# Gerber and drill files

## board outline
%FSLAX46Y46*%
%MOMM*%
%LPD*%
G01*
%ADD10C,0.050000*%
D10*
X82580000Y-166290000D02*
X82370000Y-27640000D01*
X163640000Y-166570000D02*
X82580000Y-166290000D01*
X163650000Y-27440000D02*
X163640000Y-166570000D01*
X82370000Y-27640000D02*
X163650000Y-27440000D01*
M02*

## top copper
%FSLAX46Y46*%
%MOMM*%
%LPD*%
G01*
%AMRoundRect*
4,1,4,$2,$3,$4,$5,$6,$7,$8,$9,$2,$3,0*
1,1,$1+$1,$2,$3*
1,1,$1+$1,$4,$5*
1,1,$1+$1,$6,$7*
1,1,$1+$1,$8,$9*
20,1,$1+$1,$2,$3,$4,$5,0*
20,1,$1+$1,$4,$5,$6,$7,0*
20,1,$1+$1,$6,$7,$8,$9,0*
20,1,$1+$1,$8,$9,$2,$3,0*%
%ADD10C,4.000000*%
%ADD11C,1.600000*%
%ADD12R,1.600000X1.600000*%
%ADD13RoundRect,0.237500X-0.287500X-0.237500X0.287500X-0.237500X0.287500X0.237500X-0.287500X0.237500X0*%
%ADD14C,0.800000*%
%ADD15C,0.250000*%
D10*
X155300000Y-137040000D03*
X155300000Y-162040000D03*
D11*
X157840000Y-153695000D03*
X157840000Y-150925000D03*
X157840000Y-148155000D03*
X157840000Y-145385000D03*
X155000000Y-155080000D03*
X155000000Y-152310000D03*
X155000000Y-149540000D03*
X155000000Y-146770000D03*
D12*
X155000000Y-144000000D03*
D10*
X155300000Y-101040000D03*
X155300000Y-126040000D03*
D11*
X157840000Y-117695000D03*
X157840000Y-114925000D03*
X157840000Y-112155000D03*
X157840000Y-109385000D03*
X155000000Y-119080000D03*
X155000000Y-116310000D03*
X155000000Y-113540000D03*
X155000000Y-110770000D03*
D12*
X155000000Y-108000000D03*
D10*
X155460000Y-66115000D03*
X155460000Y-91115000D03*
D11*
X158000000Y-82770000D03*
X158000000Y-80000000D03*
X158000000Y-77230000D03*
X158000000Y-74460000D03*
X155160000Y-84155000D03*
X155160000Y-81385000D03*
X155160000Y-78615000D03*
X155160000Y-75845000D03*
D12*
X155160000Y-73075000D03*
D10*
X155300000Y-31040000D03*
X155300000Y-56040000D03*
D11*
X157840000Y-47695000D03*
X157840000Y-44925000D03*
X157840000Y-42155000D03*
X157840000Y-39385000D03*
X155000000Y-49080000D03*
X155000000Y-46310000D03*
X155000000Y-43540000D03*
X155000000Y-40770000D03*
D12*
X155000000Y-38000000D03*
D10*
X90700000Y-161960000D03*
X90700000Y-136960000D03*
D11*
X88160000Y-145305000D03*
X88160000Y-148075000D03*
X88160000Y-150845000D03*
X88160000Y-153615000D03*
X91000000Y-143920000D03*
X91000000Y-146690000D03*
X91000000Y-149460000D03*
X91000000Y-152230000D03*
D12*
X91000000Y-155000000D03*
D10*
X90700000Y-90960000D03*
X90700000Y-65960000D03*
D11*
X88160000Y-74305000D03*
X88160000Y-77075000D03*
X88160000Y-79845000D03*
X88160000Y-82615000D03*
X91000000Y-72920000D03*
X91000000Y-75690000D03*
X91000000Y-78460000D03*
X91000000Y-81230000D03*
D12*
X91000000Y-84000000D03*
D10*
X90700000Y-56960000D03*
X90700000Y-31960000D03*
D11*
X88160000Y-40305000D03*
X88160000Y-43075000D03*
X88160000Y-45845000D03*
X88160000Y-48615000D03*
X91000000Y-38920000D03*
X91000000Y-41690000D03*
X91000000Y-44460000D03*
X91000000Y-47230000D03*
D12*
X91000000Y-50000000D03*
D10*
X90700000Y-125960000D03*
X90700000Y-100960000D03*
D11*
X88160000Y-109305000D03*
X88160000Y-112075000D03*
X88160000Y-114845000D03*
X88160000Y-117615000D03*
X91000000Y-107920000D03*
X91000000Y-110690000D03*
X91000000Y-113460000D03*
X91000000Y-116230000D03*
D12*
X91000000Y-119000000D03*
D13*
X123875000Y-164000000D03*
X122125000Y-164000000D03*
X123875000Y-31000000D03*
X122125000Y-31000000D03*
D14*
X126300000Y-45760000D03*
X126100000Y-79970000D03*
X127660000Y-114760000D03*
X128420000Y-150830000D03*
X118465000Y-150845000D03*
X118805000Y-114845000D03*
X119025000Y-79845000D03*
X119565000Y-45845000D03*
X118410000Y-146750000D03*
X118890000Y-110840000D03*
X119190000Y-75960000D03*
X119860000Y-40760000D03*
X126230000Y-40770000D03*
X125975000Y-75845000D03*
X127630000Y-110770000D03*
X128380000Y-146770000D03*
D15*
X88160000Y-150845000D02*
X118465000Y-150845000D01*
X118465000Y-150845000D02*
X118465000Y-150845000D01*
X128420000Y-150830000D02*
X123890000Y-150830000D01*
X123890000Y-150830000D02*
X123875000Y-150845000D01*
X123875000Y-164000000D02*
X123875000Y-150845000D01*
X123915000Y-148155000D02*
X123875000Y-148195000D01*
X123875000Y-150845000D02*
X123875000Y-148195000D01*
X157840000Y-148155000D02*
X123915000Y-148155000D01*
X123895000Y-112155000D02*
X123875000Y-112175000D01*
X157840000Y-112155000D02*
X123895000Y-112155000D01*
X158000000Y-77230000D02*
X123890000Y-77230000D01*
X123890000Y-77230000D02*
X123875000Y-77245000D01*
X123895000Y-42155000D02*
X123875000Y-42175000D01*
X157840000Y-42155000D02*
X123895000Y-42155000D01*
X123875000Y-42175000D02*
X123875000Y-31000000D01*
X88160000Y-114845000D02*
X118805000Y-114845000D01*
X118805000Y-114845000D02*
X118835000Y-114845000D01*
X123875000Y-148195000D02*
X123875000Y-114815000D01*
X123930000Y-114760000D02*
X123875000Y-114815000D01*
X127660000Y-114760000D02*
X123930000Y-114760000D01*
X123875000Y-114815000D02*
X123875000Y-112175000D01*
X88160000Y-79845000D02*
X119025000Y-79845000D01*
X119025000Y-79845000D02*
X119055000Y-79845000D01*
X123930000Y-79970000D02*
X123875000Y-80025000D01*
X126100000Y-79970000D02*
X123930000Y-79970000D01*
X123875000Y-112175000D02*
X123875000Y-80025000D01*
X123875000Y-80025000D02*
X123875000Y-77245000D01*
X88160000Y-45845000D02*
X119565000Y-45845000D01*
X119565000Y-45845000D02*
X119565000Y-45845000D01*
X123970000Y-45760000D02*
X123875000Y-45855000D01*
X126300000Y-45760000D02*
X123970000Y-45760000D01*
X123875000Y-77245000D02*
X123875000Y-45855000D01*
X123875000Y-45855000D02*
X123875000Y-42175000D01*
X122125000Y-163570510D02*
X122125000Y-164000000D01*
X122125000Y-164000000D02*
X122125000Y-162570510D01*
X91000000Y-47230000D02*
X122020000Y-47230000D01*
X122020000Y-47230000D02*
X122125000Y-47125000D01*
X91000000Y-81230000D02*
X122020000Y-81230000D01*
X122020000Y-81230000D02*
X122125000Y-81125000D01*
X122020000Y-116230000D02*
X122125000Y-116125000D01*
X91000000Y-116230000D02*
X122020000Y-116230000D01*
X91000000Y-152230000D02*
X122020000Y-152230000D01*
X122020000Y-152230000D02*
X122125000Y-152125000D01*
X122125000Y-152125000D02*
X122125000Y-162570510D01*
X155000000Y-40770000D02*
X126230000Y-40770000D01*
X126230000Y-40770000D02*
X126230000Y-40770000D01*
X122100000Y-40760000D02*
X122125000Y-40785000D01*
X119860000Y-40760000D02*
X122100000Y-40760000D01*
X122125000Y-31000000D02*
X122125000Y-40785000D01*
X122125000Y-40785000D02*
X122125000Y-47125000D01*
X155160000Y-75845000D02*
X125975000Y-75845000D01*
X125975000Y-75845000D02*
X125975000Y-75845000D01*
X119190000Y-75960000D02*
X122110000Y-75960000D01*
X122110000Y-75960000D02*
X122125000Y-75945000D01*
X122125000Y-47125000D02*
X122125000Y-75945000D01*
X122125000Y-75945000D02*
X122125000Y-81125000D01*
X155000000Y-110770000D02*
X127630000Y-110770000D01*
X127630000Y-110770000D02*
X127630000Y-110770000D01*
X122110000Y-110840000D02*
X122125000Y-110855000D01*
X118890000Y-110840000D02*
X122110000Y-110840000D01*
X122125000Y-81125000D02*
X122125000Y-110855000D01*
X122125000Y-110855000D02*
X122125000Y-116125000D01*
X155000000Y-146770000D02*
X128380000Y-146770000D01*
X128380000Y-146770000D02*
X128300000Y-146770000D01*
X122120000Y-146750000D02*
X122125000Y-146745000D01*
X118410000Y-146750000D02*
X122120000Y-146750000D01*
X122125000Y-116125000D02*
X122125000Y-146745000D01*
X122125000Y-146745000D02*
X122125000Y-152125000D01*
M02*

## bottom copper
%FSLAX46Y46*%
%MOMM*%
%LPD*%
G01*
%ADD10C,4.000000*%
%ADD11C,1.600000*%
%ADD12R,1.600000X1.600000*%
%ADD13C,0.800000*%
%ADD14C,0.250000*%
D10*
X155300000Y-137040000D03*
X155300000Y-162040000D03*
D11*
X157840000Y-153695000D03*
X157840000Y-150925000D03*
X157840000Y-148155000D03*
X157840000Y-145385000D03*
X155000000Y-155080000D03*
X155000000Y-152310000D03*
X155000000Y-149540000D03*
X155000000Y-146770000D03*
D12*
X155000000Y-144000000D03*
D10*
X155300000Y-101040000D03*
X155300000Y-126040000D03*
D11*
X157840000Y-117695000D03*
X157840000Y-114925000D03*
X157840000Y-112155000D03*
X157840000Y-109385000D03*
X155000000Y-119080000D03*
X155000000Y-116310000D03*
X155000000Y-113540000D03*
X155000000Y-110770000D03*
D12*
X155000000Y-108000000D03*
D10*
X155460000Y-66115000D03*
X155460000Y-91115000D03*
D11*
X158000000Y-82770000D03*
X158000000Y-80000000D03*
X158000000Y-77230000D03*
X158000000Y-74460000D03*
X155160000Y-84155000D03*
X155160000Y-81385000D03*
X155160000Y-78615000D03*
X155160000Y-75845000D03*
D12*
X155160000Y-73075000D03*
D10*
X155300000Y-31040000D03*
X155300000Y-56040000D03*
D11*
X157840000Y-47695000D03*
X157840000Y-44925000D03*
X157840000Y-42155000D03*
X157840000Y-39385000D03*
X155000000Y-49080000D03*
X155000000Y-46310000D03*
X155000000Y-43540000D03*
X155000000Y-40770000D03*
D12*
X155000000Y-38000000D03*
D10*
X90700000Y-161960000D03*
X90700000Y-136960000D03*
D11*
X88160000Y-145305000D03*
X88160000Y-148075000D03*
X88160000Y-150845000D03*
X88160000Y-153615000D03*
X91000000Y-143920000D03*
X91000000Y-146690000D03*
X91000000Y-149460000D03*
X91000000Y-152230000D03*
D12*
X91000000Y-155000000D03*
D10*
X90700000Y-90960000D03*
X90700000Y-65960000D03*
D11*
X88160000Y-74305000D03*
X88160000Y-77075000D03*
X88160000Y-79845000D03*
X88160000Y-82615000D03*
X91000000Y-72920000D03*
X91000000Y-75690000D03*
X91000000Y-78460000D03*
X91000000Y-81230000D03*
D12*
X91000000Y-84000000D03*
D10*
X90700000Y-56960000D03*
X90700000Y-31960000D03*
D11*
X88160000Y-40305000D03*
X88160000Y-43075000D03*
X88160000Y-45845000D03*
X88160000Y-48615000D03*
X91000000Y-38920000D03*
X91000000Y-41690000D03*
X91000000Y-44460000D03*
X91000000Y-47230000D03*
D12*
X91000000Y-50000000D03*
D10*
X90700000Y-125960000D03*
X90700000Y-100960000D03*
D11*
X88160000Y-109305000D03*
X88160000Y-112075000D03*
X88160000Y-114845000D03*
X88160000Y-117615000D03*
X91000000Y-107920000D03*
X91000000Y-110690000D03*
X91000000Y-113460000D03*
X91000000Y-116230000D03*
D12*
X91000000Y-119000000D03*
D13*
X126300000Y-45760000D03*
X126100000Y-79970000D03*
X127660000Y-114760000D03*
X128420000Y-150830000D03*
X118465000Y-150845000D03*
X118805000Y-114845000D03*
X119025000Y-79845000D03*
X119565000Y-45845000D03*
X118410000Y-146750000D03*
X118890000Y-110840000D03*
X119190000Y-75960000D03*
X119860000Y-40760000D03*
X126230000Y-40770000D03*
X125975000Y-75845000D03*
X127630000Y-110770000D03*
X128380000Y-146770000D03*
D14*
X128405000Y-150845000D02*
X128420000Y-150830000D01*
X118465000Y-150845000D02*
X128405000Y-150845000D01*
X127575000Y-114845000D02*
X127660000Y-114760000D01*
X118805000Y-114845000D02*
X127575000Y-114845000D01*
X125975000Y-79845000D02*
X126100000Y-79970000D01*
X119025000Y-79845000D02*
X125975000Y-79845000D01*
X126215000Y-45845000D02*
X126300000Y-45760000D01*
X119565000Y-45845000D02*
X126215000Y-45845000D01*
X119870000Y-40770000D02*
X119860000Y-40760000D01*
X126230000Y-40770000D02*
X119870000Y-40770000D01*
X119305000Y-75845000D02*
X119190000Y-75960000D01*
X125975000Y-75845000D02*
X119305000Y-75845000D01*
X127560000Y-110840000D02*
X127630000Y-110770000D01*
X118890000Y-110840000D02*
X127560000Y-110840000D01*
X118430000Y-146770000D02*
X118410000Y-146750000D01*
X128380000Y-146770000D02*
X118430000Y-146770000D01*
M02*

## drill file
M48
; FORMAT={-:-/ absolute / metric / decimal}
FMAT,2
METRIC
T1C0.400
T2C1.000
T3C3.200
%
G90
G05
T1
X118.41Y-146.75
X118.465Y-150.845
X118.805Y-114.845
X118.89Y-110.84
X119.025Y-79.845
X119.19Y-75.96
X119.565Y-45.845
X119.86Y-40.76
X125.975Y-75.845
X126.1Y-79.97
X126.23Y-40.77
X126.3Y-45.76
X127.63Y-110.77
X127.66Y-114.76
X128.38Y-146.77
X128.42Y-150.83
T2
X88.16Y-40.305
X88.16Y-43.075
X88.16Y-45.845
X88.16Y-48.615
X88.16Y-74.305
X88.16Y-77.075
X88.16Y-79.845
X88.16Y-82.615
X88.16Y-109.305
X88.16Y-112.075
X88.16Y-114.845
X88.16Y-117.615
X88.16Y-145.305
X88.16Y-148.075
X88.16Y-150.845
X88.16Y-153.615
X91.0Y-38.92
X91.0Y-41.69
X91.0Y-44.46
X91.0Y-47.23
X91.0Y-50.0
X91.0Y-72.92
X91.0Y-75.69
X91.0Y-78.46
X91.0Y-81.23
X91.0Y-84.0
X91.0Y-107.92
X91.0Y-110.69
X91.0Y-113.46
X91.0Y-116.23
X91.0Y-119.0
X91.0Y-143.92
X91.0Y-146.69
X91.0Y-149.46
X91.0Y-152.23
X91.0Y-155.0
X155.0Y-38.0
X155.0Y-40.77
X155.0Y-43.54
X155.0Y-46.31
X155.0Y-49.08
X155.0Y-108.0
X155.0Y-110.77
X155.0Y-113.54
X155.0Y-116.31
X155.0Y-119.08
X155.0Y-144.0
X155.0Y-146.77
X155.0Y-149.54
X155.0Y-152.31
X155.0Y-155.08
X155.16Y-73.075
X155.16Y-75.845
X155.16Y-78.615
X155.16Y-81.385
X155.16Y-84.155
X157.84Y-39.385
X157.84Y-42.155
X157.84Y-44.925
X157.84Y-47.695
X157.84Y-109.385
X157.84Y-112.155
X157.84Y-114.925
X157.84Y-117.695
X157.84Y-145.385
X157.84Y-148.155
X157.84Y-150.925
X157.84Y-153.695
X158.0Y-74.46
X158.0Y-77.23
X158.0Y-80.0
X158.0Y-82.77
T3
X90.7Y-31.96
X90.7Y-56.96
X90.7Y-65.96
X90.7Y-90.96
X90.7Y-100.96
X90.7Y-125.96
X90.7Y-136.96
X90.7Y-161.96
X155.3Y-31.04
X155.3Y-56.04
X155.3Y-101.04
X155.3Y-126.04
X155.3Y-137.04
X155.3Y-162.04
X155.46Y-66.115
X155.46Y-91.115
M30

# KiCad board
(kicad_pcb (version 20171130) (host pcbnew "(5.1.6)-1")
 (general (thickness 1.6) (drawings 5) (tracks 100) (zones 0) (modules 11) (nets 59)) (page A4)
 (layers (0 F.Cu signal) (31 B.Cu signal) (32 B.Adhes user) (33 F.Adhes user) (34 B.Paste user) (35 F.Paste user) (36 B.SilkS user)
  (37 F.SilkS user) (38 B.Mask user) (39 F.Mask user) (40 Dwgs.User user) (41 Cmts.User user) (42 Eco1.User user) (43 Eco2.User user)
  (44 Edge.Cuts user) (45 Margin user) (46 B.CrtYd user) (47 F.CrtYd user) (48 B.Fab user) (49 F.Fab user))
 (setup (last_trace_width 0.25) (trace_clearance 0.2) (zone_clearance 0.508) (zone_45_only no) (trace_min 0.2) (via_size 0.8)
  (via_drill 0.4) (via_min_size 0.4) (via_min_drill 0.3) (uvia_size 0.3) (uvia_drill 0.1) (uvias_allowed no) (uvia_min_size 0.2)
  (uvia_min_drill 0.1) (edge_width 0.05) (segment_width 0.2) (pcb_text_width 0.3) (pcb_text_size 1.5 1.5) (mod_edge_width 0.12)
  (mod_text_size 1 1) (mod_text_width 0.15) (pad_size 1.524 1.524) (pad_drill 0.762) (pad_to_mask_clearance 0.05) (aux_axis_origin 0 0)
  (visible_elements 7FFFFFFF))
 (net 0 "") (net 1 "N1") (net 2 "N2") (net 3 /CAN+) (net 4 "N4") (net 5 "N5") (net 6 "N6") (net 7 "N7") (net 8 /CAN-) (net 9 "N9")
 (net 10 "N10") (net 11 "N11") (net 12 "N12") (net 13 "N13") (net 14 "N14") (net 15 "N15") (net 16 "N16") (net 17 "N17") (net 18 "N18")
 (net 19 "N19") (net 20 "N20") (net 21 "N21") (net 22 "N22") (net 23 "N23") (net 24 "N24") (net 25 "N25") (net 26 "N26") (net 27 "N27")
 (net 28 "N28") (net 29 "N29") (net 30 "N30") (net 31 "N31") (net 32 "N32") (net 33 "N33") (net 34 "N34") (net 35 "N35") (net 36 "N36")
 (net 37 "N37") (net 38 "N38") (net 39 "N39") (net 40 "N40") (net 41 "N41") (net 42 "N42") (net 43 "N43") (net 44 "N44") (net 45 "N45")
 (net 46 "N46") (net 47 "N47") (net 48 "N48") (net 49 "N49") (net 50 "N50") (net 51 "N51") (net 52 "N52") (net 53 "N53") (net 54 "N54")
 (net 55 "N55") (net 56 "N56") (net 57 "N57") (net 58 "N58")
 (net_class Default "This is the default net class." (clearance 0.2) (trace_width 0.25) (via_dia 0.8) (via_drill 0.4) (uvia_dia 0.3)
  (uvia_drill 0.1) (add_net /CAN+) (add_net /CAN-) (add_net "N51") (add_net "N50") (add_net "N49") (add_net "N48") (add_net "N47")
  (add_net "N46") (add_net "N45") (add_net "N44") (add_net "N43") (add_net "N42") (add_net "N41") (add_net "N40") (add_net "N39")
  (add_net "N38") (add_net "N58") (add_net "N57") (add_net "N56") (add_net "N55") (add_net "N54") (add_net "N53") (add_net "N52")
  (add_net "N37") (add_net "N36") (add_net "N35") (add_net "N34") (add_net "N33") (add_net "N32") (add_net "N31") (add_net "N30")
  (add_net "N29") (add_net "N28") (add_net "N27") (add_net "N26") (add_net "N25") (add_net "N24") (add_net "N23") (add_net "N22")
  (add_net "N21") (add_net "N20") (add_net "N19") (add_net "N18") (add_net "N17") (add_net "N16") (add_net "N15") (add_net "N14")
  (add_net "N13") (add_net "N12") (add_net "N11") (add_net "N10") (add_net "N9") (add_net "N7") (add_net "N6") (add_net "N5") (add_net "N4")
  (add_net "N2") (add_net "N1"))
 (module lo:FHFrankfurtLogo (layer F.Cu) (at 122.29 88.09)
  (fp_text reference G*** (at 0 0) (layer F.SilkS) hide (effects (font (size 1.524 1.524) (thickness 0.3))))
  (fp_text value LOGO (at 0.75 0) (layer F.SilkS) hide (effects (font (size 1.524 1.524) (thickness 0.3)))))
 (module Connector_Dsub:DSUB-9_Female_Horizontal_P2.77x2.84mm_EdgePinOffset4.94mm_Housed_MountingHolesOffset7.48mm (layer F.Cu)
  (at 155 144 90)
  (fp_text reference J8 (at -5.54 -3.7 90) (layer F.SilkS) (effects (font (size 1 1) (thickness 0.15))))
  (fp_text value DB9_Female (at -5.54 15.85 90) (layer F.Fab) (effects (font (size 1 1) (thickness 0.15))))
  (pad 0 thru_hole circle (at 6.96 0.3 90) (size 4 4) (drill 3.2) (layers *.Cu *.Mask))
  (pad 0 thru_hole circle (at -18.04 0.3 90) (size 4 4) (drill 3.2) (layers *.Cu *.Mask))
  (pad 9 thru_hole circle (at -9.695 2.84 90) (size 1.6 1.6) (drill 1) (layers *.Cu *.Mask) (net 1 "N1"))
  (pad 8 thru_hole circle (at -6.925 2.84 90) (size 1.6 1.6) (drill 1) (layers *.Cu *.Mask) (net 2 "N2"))
  (pad 7 thru_hole circle (at -4.155 2.84 90) (size 1.6 1.6) (drill 1) (layers *.Cu *.Mask) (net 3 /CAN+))
  (pad 6 thru_hole circle (at -1.385 2.84 90) (size 1.6 1.6) (drill 1) (layers *.Cu *.Mask) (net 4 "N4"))
  (pad 5 thru_hole circle (at -11.08 0 90) (size 1.6 1.6) (drill 1) (layers *.Cu *.Mask) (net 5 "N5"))
  (pad 4 thru_hole circle (at -8.31 0 90) (size 1.6 1.6) (drill 1) (layers *.Cu *.Mask) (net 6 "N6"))
  (pad 3 thru_hole circle (at -5.54 0 90) (size 1.6 1.6) (drill 1) (layers *.Cu *.Mask) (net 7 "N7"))
  (pad 2 thru_hole circle (at -2.77 0 90) (size 1.6 1.6) (drill 1) (layers *.Cu *.Mask) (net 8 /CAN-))
  (pad 1 thru_hole rect (at 0 0 90) (size 1.6 1.6) (drill 1) (layers *.Cu *.Mask) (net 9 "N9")))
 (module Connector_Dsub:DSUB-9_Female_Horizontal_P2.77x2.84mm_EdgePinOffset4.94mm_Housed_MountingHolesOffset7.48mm (layer F.Cu)
  (at 155 108 90)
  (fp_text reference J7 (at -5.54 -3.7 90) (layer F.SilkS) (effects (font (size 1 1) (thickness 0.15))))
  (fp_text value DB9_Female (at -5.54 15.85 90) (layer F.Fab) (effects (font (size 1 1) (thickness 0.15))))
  (pad 0 thru_hole circle (at 6.96 0.3 90) (size 4 4) (drill 3.2) (layers *.Cu *.Mask))
  (pad 0 thru_hole circle (at -18.04 0.3 90) (size 4 4) (drill 3.2) (layers *.Cu *.Mask))
  (pad 9 thru_hole circle (at -9.695 2.84 90) (size 1.6 1.6) (drill 1) (layers *.Cu *.Mask) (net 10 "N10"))
  (pad 8 thru_hole circle (at -6.925 2.84 90) (size 1.6 1.6) (drill 1) (layers *.Cu *.Mask) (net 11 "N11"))
  (pad 7 thru_hole circle (at -4.155 2.84 90) (size 1.6 1.6) (drill 1) (layers *.Cu *.Mask) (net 3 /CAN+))
  (pad 6 thru_hole circle (at -1.385 2.84 90) (size 1.6 1.6) (drill 1) (layers *.Cu *.Mask) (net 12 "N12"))
  (pad 5 thru_hole circle (at -11.08 0 90) (size 1.6 1.6) (drill 1) (layers *.Cu *.Mask) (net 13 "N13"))
  (pad 4 thru_hole circle (at -8.31 0 90) (size 1.6 1.6) (drill 1) (layers *.Cu *.Mask) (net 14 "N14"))
  (pad 3 thru_hole circle (at -5.54 0 90) (size 1.6 1.6) (drill 1) (layers *.Cu *.Mask) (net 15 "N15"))
  (pad 2 thru_hole circle (at -2.77 0 90) (size 1.6 1.6) (drill 1) (layers *.Cu *.Mask) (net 8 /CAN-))
  (pad 1 thru_hole rect (at 0 0 90) (size 1.6 1.6) (drill 1) (layers *.Cu *.Mask) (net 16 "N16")))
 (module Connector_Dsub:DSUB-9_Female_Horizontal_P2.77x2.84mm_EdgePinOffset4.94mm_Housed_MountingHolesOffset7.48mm (layer F.Cu)
  (at 155.16 73.075 90)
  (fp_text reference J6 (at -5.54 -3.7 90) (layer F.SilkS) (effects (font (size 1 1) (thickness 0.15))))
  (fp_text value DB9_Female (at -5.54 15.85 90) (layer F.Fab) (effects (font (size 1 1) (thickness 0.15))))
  (pad 0 thru_hole circle (at 6.96 0.3 90) (size 4 4) (drill 3.2) (layers *.Cu *.Mask))
  (pad 0 thru_hole circle (at -18.04 0.3 90) (size 4 4) (drill 3.2) (layers *.Cu *.Mask))
  (pad 9 thru_hole circle (at -9.695 2.84 90) (size 1.6 1.6) (drill 1) (layers *.Cu *.Mask) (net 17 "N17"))
  (pad 8 thru_hole circle (at -6.925 2.84 90) (size 1.6 1.6) (drill 1) (layers *.Cu *.Mask) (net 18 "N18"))
  (pad 7 thru_hole circle (at -4.155 2.84 90) (size 1.6 1.6) (drill 1) (layers *.Cu *.Mask) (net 3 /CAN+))
  (pad 6 thru_hole circle (at -1.385 2.84 90) (size 1.6 1.6) (drill 1) (layers *.Cu *.Mask) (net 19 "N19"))
  (pad 5 thru_hole circle (at -11.08 0 90) (size 1.6 1.6) (drill 1) (layers *.Cu *.Mask) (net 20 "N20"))
  (pad 4 thru_hole circle (at -8.31 0 90) (size 1.6 1.6) (drill 1) (layers *.Cu *.Mask) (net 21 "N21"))
  (pad 3 thru_hole circle (at -5.54 0 90) (size 1.6 1.6) (drill 1) (layers *.Cu *.Mask) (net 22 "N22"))
  (pad 2 thru_hole circle (at -2.77 0 90) (size 1.6 1.6) (drill 1) (layers *.Cu *.Mask) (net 8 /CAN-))
  (pad 1 thru_hole rect (at 0 0 90) (size 1.6 1.6) (drill 1) (layers *.Cu *.Mask) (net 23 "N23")))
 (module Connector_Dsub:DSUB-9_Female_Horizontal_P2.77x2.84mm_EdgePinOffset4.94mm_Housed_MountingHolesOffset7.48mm (layer F.Cu)
  (at 155 38 90)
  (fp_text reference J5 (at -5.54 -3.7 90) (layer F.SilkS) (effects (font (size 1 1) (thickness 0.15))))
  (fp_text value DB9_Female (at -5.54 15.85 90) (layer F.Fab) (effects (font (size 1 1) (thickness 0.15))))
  (pad 0 thru_hole circle (at 6.96 0.3 90) (size 4 4) (drill 3.2) (layers *.Cu *.Mask))
  (pad 0 thru_hole circle (at -18.04 0.3 90) (size 4 4) (drill 3.2) (layers *.Cu *.Mask))
  (pad 9 thru_hole circle (at -9.695 2.84 90) (size 1.6 1.6) (drill 1) (layers *.Cu *.Mask) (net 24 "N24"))
  (pad 8 thru_hole circle (at -6.925 2.84 90) (size 1.6 1.6) (drill 1) (layers *.Cu *.Mask) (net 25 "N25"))
  (pad 7 thru_hole circle (at -4.155 2.84 90) (size 1.6 1.6) (drill 1) (layers *.Cu *.Mask) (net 3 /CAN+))
  (pad 6 thru_hole circle (at -1.385 2.84 90) (size 1.6 1.6) (drill 1) (layers *.Cu *.Mask) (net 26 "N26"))
  (pad 5 thru_hole circle (at -11.08 0 90) (size 1.6 1.6) (drill 1) (layers *.Cu *.Mask) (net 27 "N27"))
  (pad 4 thru_hole circle (at -8.31 0 90) (size 1.6 1.6) (drill 1) (layers *.Cu *.Mask) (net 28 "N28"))
  (pad 3 thru_hole circle (at -5.54 0 90) (size 1.6 1.6) (drill 1) (layers *.Cu *.Mask) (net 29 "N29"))
  (pad 2 thru_hole circle (at -2.77 0 90) (size 1.6 1.6) (drill 1) (layers *.Cu *.Mask) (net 8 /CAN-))
  (pad 1 thru_hole rect (at 0 0 90) (size 1.6 1.6) (drill 1) (layers *.Cu *.Mask) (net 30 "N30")))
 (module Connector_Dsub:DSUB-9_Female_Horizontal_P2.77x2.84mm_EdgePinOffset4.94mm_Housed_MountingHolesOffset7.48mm (layer F.Cu)
  (at 91 155 270)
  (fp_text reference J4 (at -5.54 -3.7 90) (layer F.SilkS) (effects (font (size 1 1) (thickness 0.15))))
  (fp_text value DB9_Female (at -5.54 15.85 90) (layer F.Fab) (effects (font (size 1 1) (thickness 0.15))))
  (pad 0 thru_hole circle (at 6.96 0.3 270) (size 4 4) (drill 3.2) (layers *.Cu *.Mask))
  (pad 0 thru_hole circle (at -18.04 0.3 270) (size 4 4) (drill 3.2) (layers *.Cu *.Mask))
  (pad 9 thru_hole circle (at -9.695 2.84 270) (size 1.6 1.6) (drill 1) (layers *.Cu *.Mask) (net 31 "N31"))
  (pad 8 thru_hole circle (at -6.925 2.84 270) (size 1.6 1.6) (drill 1) (layers *.Cu *.Mask) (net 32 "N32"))
  (pad 7 thru_hole circle (at -4.155 2.84 270) (size 1.6 1.6) (drill 1) (layers *.Cu *.Mask) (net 3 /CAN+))
  (pad 6 thru_hole circle (at -1.385 2.84 270) (size 1.6 1.6) (drill 1) (layers *.Cu *.Mask) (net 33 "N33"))
  (pad 5 thru_hole circle (at -11.08 0 270) (size 1.6 1.6) (drill 1) (layers *.Cu *.Mask) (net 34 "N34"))
  (pad 4 thru_hole circle (at -8.31 0 270) (size 1.6 1.6) (drill 1) (layers *.Cu *.Mask) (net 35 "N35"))
  (pad 3 thru_hole circle (at -5.54 0 270) (size 1.6 1.6) (drill 1) (layers *.Cu *.Mask) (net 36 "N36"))
  (pad 2 thru_hole circle (at -2.77 0 270) (size 1.6 1.6) (drill 1) (layers *.Cu *.Mask) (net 8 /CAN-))
  (pad 1 thru_hole rect (at 0 0 270) (size 1.6 1.6) (drill 1) (layers *.Cu *.Mask) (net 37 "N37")))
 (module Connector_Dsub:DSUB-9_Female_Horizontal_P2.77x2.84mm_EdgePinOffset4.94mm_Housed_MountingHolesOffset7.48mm (layer F.Cu)
  (at 91 84 270)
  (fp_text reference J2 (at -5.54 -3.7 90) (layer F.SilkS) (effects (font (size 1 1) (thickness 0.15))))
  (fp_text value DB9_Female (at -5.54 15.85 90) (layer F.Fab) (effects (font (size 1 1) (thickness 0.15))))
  (pad 0 thru_hole circle (at 6.96 0.3 270) (size 4 4) (drill 3.2) (layers *.Cu *.Mask))
  (pad 0 thru_hole circle (at -18.04 0.3 270) (size 4 4) (drill 3.2) (layers *.Cu *.Mask))
  (pad 9 thru_hole circle (at -9.695 2.84 270) (size 1.6 1.6) (drill 1) (layers *.Cu *.Mask) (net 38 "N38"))
  (pad 8 thru_hole circle (at -6.925 2.84 270) (size 1.6 1.6) (drill 1) (layers *.Cu *.Mask) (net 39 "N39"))
  (pad 7 thru_hole circle (at -4.155 2.84 270) (size 1.6 1.6) (drill 1) (layers *.Cu *.Mask) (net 3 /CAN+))
  (pad 6 thru_hole circle (at -1.385 2.84 270) (size 1.6 1.6) (drill 1) (layers *.Cu *.Mask) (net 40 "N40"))
  (pad 5 thru_hole circle (at -11.08 0 270) (size 1.6 1.6) (drill 1) (layers *.Cu *.Mask) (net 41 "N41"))
  (pad 4 thru_hole circle (at -8.31 0 270) (size 1.6 1.6) (drill 1) (layers *.Cu *.Mask) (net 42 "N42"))
  (pad 3 thru_hole circle (at -5.54 0 270) (size 1.6 1.6) (drill 1) (layers *.Cu *.Mask) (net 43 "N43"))
  (pad 2 thru_hole circle (at -2.77 0 270) (size 1.6 1.6) (drill 1) (layers *.Cu *.Mask) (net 8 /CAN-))
  (pad 1 thru_hole rect (at 0 0 270) (size 1.6 1.6) (drill 1) (layers *.Cu *.Mask) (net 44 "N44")))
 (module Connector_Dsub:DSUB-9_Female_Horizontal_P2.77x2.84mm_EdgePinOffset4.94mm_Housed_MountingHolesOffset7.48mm (layer F.Cu)
  (at 91 50 270)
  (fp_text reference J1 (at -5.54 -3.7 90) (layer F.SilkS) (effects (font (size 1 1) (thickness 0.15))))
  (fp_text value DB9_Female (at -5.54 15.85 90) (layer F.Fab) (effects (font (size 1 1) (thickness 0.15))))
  (pad 0 thru_hole circle (at 6.96 0.3 270) (size 4 4) (drill 3.2) (layers *.Cu *.Mask))
  (pad 0 thru_hole circle (at -18.04 0.3 270) (size 4 4) (drill 3.2) (layers *.Cu *.Mask))
  (pad 9 thru_hole circle (at -9.695 2.84 270) (size 1.6 1.6) (drill 1) (layers *.Cu *.Mask) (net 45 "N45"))
  (pad 8 thru_hole circle (at -6.925 2.84 270) (size 1.6 1.6) (drill 1) (layers *.Cu *.Mask) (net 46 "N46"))
  (pad 7 thru_hole circle (at -4.155 2.84 270) (size 1.6 1.6) (drill 1) (layers *.Cu *.Mask) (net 3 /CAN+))
  (pad 6 thru_hole circle (at -1.385 2.84 270) (size 1.6 1.6) (drill 1) (layers *.Cu *.Mask) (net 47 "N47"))
  (pad 5 thru_hole circle (at -11.08 0 270) (size 1.6 1.6) (drill 1) (layers *.Cu *.Mask) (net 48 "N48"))
  (pad 4 thru_hole circle (at -8.31 0 270) (size 1.6 1.6) (drill 1) (layers *.Cu *.Mask) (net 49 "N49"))
  (pad 3 thru_hole circle (at -5.54 0 270) (size 1.6 1.6) (drill 1) (layers *.Cu *.Mask) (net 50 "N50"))
  (pad 2 thru_hole circle (at -2.77 0 270) (size 1.6 1.6) (drill 1) (layers *.Cu *.Mask) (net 8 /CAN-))
  (pad 1 thru_hole rect (at 0 0 270) (size 1.6 1.6) (drill 1) (layers *.Cu *.Mask) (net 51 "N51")))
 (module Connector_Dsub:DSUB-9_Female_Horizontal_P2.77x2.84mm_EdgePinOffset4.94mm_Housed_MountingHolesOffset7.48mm (layer F.Cu)
  (at 91 119 270)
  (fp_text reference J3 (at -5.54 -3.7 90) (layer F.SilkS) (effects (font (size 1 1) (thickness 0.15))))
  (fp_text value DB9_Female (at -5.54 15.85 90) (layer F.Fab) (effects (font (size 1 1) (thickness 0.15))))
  (pad 0 thru_hole circle (at 6.96 0.3 270) (size 4 4) (drill 3.2) (layers *.Cu *.Mask))
  (pad 0 thru_hole circle (at -18.04 0.3 270) (size 4 4) (drill 3.2) (layers *.Cu *.Mask))
  (pad 9 thru_hole circle (at -9.695 2.84 270) (size 1.6 1.6) (drill 1) (layers *.Cu *.Mask) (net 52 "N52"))
  (pad 8 thru_hole circle (at -6.925 2.84 270) (size 1.6 1.6) (drill 1) (layers *.Cu *.Mask) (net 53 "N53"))
  (pad 7 thru_hole circle (at -4.155 2.84 270) (size 1.6 1.6) (drill 1) (layers *.Cu *.Mask) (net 3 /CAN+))
  (pad 6 thru_hole circle (at -1.385 2.84 270) (size 1.6 1.6) (drill 1) (layers *.Cu *.Mask) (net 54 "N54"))
  (pad 5 thru_hole circle (at -11.08 0 270) (size 1.6 1.6) (drill 1) (layers *.Cu *.Mask) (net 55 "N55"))
  (pad 4 thru_hole circle (at -8.31 0 270) (size 1.6 1.6) (drill 1) (layers *.Cu *.Mask) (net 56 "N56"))
  (pad 3 thru_hole circle (at -5.54 0 270) (size 1.6 1.6) (drill 1) (layers *.Cu *.Mask) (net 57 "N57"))
  (pad 2 thru_hole circle (at -2.77 0 270) (size 1.6 1.6) (drill 1) (layers *.Cu *.Mask) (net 8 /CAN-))
  (pad 1 thru_hole rect (at 0 0 270) (size 1.6 1.6) (drill 1) (layers *.Cu *.Mask) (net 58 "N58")))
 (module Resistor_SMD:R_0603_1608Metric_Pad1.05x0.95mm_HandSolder (layer F.Cu) (at 123 164)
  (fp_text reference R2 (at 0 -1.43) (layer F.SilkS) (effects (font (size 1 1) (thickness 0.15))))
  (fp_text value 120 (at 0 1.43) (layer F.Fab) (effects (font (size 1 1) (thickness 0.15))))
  (pad 2 smd roundrect (at 0.875 0) (size 1.05 0.95) (layers F.Cu F.Paste F.Mask) (roundrect_rratio 0.25) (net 3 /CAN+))
  (pad 1 smd roundrect (at -0.875 0) (size 1.05 0.95) (layers F.Cu F.Paste F.Mask) (roundrect_rratio 0.25) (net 8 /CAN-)))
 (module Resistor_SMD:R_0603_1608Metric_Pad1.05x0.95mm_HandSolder (layer F.Cu) (at 123 31)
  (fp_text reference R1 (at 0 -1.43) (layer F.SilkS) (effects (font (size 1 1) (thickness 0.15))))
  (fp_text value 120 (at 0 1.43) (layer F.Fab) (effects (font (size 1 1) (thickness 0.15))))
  (pad 2 smd roundrect (at 0.875 0) (size 1.05 0.95) (layers F.Cu F.Paste F.Mask) (roundrect_rratio 0.25) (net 3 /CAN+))
  (pad 1 smd roundrect (at -0.875 0) (size 1.05 0.95) (layers F.Cu F.Paste F.Mask) (roundrect_rratio 0.25) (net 8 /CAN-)))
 (gr_line (start 82.58 166.29) (end 82.37 27.64) (layer Edge.Cuts) (width 0.05))
 (gr_line (start 163.64 166.57) (end 82.58 166.29) (layer Edge.Cuts) (width 0.05))
 (gr_line (start 163.65 27.44) (end 163.64 166.57) (layer Edge.Cuts) (width 0.05))
 (gr_line (start 82.37 27.64) (end 163.65 27.44) (layer Edge.Cuts) (width 0.05))
 (via (at 126.3 45.76) (size 0.8) (drill 0.4) (layers F.Cu B.Cu) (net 3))
 (via (at 126.1 79.97) (size 0.8) (drill 0.4) (layers F.Cu B.Cu) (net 3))
 (via (at 127.66 114.76) (size 0.8) (drill 0.4) (layers F.Cu B.Cu) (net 3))
 (via (at 128.42 150.83) (size 0.8) (drill 0.4) (layers F.Cu B.Cu) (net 3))
 (segment (start 88.16 150.845) (end 118.465 150.845) (width 0.25) (layer F.Cu) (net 3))
 (segment (start 118.465 150.845) (end 118.465 150.845) (width 0.25) (layer F.Cu) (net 3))
 (via (at 118.465 150.845) (size 0.8) (drill 0.4) (layers F.Cu B.Cu) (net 3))
 (segment (start 128.405 150.845) (end 128.42 150.83) (width 0.25) (layer B.Cu) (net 3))
 (segment (start 118.465 150.845) (end 128.405 150.845) (width 0.25) (layer B.Cu) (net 3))
 (segment (start 128.42 150.83) (end 123.89 150.83) (width 0.25) (layer F.Cu) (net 3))
 (segment (start 123.89 150.83) (end 123.875 150.845) (width 0.25) (layer F.Cu) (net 3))
 (segment (start 123.875 164) (end 123.875 150.845) (width 0.25) (layer F.Cu) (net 3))
 (segment (start 123.915 148.155) (end 123.875 148.195) (width 0.25) (layer F.Cu) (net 3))
 (segment (start 123.875 150.845) (end 123.875 148.195) (width 0.25) (layer F.Cu) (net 3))
 (segment (start 157.84 148.155) (end 123.915 148.155) (width 0.25) (layer F.Cu) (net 3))
 (segment (start 123.895 112.155) (end 123.875 112.175) (width 0.25) (layer F.Cu) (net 3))
 (segment (start 157.84 112.155) (end 123.895 112.155) (width 0.25) (layer F.Cu) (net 3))
 (segment (start 158 77.23) (end 123.89 77.23) (width 0.25) (layer F.Cu) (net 3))
 (segment (start 123.89 77.23) (end 123.875 77.245) (width 0.25) (layer F.Cu) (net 3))
 (segment (start 123.895 42.155) (end 123.875 42.175) (width 0.25) (layer F.Cu) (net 3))
 (segment (start 157.84 42.155) (end 123.895 42.155) (width 0.25) (layer F.Cu) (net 3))
 (segment (start 123.875 42.175) (end 123.875 31) (width 0.25) (layer F.Cu) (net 3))
 (segment (start 88.16 114.845) (end 118.805 114.845) (width 0.25) (layer F.Cu) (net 3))
 (segment (start 118.805 114.845) (end 118.835 114.845) (width 0.25) (layer F.Cu) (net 3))
 (via (at 118.805 114.845) (size 0.8) (drill 0.4) (layers F.Cu B.Cu) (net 3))
 (segment (start 127.575 114.845) (end 127.66 114.76) (width 0.25) (layer B.Cu) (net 3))
 (segment (start 118.805 114.845) (end 127.575 114.845) (width 0.25) (layer B.Cu) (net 3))
 (segment (start 123.875 148.195) (end 123.875 114.815) (width 0.25) (layer F.Cu) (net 3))
 (segment (start 123.93 114.76) (end 123.875 114.815) (width 0.25) (layer F.Cu) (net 3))
 (segment (start 127.66 114.76) (end 123.93 114.76) (width 0.25) (layer F.Cu) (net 3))
 (segment (start 123.875 114.815) (end 123.875 112.175) (width 0.25) (layer F.Cu) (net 3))
 (segment (start 88.16 79.845) (end 119.025 79.845) (width 0.25) (layer F.Cu) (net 3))
 (segment (start 119.025 79.845) (end 119.055 79.845) (width 0.25) (layer F.Cu) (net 3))
 (via (at 119.025 79.845) (size 0.8) (drill 0.4) (layers F.Cu B.Cu) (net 3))
 (segment (start 123.93 79.97) (end 123.875 80.025) (width 0.25) (layer F.Cu) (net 3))
 (segment (start 126.1 79.97) (end 123.93 79.97) (width 0.25) (layer F.Cu) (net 3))
 (segment (start 123.875 112.175) (end 123.875 80.025) (width 0.25) (layer F.Cu) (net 3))
 (segment (start 123.875 80.025) (end 123.875 77.245) (width 0.25) (layer F.Cu) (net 3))
 (segment (start 125.975 79.845) (end 126.1 79.97) (width 0.25) (layer B.Cu) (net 3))
 (segment (start 119.025 79.845) (end 125.975 79.845) (width 0.25) (layer B.Cu) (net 3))
 (segment (start 88.16 45.845) (end 119.565 45.845) (width 0.25) (layer F.Cu) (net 3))
 (segment (start 119.565 45.845) (end 119.565 45.845) (width 0.25) (layer F.Cu) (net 3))
 (via (at 119.565 45.845) (size 0.8) (drill 0.4) (layers F.Cu B.Cu) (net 3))
 (segment (start 126.215 45.845) (end 126.3 45.76) (width 0.25) (layer B.Cu) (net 3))
 (segment (start 119.565 45.845) (end 126.215 45.845) (width 0.25) (layer B.Cu) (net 3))
 (segment (start 123.97 45.76) (end 123.875 45.855) (width 0.25) (layer F.Cu) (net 3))
 (segment (start 126.3 45.76) (end 123.97 45.76) (width 0.25) (layer F.Cu) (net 3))
 (segment (start 123.875 77.245) (end 123.875 45.855) (width 0.25) (layer F.Cu) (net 3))
 (segment (start 123.875 45.855) (end 123.875 42.175) (width 0.25) (layer F.Cu) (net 3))
 (via (at 118.41 146.75) (size 0.8) (drill 0.4) (layers F.Cu B.Cu) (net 8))
 (via (at 118.89 110.84) (size 0.8) (drill 0.4) (layers F.Cu B.Cu) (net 8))
 (via (at 119.19 75.96) (size 0.8) (drill 0.4) (layers F.Cu B.Cu) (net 8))
 (via (at 119.86 40.76) (size 0.8) (drill 0.4) (layers F.Cu B.Cu) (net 8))
 (segment (start 122.125 163.57051) (end 122.125 164) (width 0.25) (layer F.Cu) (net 8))
 (segment (start 122.125 164) (end 122.125 162.57051) (width 0.25) (layer F.Cu) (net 8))
 (segment (start 91 47.23) (end 122.02 47.23) (width 0.25) (layer F.Cu) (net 8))
 (segment (start 122.02 47.23) (end 122.125 47.125) (width 0.25) (layer F.Cu) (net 8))
 (segment (start 91 81.23) (end 122.02 81.23) (width 0.25) (layer F.Cu) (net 8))
 (segment (start 122.02 81.23) (end 122.125 81.125) (width 0.25) (layer F.Cu) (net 8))
 (segment (start 122.02 116.23) (end 122.125 116.125) (width 0.25) (layer F.Cu) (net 8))
 (segment (start 91 116.23) (end 122.02 116.23) (width 0.25) (layer F.Cu) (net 8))
 (segment (start 91 152.23) (end 122.02 152.23) (width 0.25) (layer F.Cu) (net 8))
 (segment (start 122.02 152.23) (end 122.125 152.125) (width 0.25) (layer F.Cu) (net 8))
 (segment (start 122.125 152.125) (end 122.125 162.57051) (width 0.25) (layer F.Cu) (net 8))
 (segment (start 155 40.77) (end 126.23 40.77) (width 0.25) (layer F.Cu) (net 8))
 (segment (start 126.23 40.77) (end 126.23 40.77) (width 0.25) (layer F.Cu) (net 8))
 (via (at 126.23 40.77) (size 0.8) (drill 0.4) (layers F.Cu B.Cu) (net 8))
 (segment (start 119.87 40.77) (end 119.86 40.76) (width 0.25) (layer B.Cu) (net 8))
 (segment (start 126.23 40.77) (end 119.87 40.77) (width 0.25) (layer B.Cu) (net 8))
 (segment (start 122.1 40.76) (end 122.125 40.785) (width 0.25) (layer F.Cu) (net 8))
 (segment (start 119.86 40.76) (end 122.1 40.76) (width 0.25) (layer F.Cu) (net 8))
 (segment (start 122.125 31) (end 122.125 40.785) (width 0.25) (layer F.Cu) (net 8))
 (segment (start 122.125 40.785) (end 122.125 47.125) (width 0.25) (layer F.Cu) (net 8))
 (segment (start 155.16 75.845) (end 125.975 75.845) (width 0.25) (layer F.Cu) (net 8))
 (segment (start 125.975 75.845) (end 125.975 75.845) (width 0.25) (layer F.Cu) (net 8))
 (via (at 125.975 75.845) (size 0.8) (drill 0.4) (layers F.Cu B.Cu) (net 8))
 (segment (start 119.305 75.845) (end 119.19 75.96) (width 0.25) (layer B.Cu) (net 8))
 (segment (start 125.975 75.845) (end 119.305 75.845) (width 0.25) (layer B.Cu) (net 8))
 (segment (start 119.19 75.96) (end 122.11 75.96) (width 0.25) (layer F.Cu) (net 8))
 (segment (start 122.11 75.96) (end 122.125 75.945) (width 0.25) (layer F.Cu) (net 8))
 (segment (start 122.125 47.125) (end 122.125 75.945) (width 0.25) (layer F.Cu) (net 8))
 (segment (start 122.125 75.945) (end 122.125 81.125) (width 0.25) (layer F.Cu) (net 8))
 (segment (start 155 110.77) (end 127.63 110.77) (width 0.25) (layer F.Cu) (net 8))
 (segment (start 127.63 110.77) (end 127.63 110.77) (width 0.25) (layer F.Cu) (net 8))
 (via (at 127.63 110.77) (size 0.8) (drill 0.4) (layers F.Cu B.Cu) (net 8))
 (segment (start 122.11 110.84) (end 122.125 110.855) (width 0.25) (layer F.Cu) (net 8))
 (segment (start 118.89 110.84) (end 122.11 110.84) (width 0.25) (layer F.Cu) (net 8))
 (segment (start 122.125 81.125) (end 122.125 110.855) (width 0.25) (layer F.Cu) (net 8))
 (segment (start 122.125 110.855) (end 122.125 116.125) (width 0.25) (layer F.Cu) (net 8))
 (segment (start 127.56 110.84) (end 127.63 110.77) (width 0.25) (layer B.Cu) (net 8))
 (segment (start 118.89 110.84) (end 127.56 110.84) (width 0.25) (layer B.Cu) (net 8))
 (segment (start 155 146.77) (end 128.38 146.77) (width 0.25) (layer F.Cu) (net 8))
 (segment (start 128.38 146.77) (end 128.3 146.77) (width 0.25) (layer F.Cu) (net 8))
 (via (at 128.38 146.77) (size 0.8) (drill 0.4) (layers F.Cu B.Cu) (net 8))
 (segment (start 118.43 146.77) (end 118.41 146.75) (width 0.25) (layer B.Cu) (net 8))
 (segment (start 128.38 146.77) (end 118.43 146.77) (width 0.25) (layer B.Cu) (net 8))
 (segment (start 122.12 146.75) (end 122.125 146.745) (width 0.25) (layer F.Cu) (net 8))
 (segment (start 118.41 146.75) (end 122.12 146.75) (width 0.25) (layer F.Cu) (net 8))
 (segment (start 122.125 116.125) (end 122.125 146.745) (width 0.25) (layer F.Cu) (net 8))
 (segment (start 122.125 146.745) (end 122.125 152.125) (width 0.25) (layer F.Cu) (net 8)))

